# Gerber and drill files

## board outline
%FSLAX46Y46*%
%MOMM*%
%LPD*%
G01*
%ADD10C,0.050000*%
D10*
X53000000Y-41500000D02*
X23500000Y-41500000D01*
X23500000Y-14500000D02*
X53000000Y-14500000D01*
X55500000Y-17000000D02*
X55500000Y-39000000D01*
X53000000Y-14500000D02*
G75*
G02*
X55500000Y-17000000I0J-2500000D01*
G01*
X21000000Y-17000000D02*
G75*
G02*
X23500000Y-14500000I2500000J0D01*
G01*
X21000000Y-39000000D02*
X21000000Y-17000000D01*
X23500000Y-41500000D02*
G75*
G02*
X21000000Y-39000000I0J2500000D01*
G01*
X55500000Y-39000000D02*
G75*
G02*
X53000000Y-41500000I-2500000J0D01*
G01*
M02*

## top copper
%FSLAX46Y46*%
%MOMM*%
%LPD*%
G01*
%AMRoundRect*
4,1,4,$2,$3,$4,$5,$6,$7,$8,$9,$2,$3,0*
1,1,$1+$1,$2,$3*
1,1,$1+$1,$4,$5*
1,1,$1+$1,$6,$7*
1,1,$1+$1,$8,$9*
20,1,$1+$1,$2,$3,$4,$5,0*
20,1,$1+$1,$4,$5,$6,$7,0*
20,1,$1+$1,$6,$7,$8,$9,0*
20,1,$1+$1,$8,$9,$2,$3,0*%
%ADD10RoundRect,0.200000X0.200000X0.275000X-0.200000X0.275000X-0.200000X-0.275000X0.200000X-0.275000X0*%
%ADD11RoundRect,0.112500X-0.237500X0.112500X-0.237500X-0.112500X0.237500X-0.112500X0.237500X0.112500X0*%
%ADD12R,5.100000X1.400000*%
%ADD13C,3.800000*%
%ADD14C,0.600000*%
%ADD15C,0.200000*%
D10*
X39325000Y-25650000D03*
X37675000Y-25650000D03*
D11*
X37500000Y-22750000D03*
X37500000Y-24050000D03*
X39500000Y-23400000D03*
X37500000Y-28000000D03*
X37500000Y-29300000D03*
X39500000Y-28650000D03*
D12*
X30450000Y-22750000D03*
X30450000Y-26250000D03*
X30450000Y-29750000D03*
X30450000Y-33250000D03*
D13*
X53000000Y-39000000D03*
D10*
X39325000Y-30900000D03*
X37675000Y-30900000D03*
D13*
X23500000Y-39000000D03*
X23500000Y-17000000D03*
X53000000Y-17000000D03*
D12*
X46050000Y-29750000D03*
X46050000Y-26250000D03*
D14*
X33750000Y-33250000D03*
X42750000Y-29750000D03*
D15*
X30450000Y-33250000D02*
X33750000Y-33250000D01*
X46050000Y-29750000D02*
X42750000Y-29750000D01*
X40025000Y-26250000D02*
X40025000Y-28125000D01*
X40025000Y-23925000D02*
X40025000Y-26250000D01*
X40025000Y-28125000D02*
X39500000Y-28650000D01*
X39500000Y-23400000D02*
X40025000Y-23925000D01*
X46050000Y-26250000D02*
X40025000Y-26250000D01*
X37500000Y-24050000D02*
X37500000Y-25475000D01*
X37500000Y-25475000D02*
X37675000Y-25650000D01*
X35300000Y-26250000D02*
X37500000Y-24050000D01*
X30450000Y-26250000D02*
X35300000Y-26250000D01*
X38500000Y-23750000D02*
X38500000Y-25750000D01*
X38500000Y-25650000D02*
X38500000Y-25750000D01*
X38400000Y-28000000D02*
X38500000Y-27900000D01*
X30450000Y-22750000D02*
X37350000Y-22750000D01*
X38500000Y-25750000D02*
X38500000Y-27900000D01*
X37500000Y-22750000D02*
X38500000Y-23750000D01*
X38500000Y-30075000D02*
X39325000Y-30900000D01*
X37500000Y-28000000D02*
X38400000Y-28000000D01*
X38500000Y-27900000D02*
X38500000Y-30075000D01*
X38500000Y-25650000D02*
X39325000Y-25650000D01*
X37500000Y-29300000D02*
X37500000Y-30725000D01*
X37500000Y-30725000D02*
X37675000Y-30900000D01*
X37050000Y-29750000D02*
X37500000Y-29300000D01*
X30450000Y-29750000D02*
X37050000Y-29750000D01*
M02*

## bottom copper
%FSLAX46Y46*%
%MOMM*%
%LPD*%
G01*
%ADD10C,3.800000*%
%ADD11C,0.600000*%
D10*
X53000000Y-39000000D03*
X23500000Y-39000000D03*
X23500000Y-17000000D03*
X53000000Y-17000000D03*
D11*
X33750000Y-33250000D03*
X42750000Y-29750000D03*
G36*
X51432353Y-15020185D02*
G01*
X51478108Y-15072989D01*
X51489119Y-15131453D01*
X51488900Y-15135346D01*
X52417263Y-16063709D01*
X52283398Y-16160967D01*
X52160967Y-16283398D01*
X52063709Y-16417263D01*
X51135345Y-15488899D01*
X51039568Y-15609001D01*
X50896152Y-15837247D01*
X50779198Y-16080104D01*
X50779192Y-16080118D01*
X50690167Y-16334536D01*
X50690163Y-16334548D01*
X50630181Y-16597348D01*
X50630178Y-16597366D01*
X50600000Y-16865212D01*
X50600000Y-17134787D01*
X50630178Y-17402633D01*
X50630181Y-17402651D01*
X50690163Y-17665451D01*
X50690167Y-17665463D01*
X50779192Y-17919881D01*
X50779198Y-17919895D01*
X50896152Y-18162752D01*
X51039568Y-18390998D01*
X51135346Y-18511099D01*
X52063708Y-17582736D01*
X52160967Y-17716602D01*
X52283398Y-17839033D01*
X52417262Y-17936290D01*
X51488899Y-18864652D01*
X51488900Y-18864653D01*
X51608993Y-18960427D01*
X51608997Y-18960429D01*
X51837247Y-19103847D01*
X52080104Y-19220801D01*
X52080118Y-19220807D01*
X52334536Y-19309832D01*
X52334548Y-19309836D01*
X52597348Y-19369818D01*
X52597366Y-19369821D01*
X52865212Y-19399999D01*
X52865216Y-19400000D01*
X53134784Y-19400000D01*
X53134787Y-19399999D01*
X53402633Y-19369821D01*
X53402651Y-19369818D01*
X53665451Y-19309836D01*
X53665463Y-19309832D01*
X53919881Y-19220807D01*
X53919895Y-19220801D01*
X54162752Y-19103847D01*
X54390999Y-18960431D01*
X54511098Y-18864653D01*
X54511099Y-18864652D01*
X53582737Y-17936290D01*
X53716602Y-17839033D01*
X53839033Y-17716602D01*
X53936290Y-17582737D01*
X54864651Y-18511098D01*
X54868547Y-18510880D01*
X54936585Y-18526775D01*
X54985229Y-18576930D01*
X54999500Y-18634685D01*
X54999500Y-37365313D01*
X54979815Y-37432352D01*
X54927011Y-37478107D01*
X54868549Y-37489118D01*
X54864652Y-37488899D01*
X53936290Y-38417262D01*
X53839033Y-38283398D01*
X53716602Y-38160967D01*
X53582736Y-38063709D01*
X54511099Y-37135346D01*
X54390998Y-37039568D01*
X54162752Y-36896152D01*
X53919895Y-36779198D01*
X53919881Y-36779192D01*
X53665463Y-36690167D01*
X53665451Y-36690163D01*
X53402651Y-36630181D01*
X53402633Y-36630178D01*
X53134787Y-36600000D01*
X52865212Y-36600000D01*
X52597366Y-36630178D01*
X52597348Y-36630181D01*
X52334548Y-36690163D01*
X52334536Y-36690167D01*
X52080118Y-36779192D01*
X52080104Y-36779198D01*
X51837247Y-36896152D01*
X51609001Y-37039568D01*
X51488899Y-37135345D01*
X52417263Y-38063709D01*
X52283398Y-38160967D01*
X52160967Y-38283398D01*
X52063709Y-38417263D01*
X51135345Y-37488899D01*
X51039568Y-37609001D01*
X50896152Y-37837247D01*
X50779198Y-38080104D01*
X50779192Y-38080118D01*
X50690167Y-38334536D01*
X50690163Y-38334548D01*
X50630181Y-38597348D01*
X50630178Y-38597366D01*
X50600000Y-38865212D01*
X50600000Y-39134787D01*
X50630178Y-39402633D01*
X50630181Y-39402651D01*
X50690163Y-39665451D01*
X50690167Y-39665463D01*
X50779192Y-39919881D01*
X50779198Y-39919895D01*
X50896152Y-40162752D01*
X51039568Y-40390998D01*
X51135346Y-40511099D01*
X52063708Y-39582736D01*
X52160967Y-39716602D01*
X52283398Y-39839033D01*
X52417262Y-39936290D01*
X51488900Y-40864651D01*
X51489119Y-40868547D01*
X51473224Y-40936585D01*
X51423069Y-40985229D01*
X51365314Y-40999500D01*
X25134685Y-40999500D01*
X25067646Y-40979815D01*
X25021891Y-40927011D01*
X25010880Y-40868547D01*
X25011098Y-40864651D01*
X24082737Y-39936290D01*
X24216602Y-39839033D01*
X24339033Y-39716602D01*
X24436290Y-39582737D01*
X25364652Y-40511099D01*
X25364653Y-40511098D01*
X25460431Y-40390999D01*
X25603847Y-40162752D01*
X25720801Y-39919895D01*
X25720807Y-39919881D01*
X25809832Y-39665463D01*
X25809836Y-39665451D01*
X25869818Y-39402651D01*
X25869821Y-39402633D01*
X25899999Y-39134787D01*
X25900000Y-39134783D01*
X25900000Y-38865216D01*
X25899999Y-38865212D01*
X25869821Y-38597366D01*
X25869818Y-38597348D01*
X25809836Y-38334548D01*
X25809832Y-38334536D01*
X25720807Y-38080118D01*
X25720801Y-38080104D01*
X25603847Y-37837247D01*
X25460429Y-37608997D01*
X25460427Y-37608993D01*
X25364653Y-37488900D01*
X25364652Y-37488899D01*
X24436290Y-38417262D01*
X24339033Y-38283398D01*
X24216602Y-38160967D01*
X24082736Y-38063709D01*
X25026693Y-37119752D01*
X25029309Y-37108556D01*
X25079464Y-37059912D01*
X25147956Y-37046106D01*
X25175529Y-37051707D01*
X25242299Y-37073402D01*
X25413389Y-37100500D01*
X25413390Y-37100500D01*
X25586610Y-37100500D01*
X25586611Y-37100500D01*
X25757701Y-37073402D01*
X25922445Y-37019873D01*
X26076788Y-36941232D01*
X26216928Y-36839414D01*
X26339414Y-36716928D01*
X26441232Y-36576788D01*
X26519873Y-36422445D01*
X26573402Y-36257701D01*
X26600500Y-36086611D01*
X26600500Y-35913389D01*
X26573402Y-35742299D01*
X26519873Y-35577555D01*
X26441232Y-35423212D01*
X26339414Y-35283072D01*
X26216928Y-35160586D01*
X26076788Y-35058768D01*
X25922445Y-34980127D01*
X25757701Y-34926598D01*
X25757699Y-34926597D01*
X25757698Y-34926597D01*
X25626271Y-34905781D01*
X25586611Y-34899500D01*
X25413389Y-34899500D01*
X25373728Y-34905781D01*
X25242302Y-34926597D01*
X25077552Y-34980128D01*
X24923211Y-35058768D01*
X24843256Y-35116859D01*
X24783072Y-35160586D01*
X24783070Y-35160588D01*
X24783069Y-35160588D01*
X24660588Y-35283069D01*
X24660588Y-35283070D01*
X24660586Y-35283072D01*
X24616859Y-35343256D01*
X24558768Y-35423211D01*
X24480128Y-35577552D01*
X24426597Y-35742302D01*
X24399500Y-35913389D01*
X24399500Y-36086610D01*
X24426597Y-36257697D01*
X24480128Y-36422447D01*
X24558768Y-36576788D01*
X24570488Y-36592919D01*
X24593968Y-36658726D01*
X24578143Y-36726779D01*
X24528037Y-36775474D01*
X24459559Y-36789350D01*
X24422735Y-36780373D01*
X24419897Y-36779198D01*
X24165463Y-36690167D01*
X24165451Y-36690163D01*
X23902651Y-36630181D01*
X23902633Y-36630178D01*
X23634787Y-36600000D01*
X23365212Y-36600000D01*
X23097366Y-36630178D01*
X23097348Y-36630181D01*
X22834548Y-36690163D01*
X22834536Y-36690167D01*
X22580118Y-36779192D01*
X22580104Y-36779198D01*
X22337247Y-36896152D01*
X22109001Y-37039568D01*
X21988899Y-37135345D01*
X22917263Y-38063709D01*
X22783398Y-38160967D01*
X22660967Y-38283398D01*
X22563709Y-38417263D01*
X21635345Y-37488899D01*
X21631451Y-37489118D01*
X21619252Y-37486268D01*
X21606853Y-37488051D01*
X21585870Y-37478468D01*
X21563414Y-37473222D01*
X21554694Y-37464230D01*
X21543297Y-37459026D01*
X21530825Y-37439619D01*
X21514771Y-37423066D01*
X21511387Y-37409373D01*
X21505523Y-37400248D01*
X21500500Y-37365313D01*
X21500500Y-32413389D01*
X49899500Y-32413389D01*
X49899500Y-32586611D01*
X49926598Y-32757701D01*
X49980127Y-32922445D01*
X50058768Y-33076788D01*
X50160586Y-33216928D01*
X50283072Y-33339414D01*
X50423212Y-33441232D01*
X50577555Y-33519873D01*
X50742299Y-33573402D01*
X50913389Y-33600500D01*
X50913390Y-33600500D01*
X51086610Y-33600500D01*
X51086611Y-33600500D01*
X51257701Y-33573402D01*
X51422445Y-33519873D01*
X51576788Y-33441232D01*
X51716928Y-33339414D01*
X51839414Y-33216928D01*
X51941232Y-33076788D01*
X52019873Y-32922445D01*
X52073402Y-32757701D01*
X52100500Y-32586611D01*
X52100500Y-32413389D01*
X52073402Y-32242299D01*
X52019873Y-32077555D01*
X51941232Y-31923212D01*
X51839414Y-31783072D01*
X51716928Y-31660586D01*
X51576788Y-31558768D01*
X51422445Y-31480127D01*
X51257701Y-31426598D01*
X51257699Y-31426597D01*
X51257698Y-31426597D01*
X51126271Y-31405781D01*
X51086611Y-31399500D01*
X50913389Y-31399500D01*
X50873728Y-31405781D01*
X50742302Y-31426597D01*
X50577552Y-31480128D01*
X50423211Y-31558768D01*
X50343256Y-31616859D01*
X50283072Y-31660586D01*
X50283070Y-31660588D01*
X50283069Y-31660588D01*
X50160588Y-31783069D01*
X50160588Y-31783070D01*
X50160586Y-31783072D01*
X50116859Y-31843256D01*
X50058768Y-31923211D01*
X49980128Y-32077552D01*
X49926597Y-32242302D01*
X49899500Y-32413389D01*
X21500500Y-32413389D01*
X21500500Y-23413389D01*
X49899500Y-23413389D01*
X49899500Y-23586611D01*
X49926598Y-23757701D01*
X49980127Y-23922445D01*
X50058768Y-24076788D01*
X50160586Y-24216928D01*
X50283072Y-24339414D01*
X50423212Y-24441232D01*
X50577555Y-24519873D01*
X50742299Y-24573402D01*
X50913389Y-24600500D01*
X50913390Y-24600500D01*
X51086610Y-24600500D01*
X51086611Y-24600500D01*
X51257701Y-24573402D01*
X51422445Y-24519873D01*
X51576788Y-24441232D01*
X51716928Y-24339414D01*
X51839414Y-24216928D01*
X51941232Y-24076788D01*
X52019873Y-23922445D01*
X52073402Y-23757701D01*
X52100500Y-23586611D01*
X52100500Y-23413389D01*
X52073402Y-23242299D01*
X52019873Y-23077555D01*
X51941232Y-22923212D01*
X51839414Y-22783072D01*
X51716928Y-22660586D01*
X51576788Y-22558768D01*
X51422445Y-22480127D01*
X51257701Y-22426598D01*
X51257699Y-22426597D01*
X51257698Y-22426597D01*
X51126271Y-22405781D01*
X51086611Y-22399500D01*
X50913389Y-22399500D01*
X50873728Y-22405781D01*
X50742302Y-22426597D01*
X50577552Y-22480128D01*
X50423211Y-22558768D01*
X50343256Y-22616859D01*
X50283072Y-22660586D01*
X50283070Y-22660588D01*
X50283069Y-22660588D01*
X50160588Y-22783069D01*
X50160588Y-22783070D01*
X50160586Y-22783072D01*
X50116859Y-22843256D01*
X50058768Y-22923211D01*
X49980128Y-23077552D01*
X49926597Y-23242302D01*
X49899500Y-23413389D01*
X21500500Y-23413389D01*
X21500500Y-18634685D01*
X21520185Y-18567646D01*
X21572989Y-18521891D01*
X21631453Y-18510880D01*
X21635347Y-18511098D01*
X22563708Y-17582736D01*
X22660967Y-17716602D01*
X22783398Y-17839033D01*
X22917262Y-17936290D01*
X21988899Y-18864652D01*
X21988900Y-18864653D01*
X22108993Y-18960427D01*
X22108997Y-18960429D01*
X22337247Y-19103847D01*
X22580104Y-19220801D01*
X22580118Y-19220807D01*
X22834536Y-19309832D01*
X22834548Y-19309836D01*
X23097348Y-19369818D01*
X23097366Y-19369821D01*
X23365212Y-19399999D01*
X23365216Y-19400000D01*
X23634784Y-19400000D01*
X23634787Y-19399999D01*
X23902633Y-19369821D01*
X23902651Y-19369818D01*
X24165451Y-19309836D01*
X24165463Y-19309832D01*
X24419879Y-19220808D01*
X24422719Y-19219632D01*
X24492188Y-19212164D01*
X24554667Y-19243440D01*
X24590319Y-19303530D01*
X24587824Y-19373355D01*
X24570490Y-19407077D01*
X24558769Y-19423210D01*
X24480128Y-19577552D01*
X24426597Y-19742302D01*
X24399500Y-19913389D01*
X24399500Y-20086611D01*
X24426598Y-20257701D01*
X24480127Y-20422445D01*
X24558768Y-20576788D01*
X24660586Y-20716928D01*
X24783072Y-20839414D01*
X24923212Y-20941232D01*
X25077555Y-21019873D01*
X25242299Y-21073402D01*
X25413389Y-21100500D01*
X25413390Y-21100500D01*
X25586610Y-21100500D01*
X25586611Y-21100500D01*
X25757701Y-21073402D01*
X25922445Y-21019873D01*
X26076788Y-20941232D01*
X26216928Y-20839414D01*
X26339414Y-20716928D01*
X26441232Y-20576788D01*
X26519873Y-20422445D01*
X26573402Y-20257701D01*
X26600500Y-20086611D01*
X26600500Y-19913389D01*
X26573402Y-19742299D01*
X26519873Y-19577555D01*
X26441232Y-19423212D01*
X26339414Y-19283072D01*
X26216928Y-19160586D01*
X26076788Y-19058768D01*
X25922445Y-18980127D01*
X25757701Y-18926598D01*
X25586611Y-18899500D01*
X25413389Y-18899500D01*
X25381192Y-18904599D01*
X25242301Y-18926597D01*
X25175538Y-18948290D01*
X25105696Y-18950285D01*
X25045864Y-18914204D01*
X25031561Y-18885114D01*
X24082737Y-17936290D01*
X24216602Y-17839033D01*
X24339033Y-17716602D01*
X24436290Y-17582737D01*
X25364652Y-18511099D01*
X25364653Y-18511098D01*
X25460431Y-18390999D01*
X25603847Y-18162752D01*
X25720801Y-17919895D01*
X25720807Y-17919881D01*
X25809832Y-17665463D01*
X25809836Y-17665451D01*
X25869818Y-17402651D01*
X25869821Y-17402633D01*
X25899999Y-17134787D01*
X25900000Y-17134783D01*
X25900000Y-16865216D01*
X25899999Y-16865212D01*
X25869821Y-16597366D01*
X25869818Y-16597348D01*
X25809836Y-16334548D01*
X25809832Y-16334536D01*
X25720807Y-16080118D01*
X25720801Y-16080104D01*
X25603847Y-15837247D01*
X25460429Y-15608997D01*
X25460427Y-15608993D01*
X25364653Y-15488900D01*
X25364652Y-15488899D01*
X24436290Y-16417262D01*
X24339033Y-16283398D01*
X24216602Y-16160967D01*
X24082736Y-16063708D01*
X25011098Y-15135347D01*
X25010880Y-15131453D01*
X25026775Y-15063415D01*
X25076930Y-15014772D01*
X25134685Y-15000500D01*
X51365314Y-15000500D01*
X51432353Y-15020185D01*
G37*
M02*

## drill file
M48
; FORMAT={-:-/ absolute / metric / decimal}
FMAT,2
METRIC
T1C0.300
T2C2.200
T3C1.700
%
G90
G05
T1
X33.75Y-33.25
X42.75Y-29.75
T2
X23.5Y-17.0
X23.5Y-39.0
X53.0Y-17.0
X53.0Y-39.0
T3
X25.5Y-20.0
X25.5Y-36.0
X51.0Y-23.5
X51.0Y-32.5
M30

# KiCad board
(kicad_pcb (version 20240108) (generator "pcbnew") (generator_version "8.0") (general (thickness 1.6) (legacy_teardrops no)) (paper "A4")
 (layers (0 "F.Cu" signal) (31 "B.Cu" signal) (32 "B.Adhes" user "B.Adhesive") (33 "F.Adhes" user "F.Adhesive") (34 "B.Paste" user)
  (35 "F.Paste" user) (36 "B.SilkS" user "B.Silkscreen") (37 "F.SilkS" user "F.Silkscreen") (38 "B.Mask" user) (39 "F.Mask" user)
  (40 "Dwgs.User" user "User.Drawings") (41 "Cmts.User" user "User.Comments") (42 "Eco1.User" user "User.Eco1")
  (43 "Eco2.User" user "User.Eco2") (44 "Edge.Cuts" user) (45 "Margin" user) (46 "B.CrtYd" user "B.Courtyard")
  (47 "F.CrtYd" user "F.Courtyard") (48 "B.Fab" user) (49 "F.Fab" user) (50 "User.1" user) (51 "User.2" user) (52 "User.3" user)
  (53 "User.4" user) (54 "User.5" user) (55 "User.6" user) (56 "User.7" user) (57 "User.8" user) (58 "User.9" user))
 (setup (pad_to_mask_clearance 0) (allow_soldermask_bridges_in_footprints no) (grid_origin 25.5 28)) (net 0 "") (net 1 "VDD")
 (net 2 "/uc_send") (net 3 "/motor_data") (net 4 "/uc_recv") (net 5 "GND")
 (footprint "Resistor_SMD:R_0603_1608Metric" (layer "F.Cu") (at 38.5 25.65 180)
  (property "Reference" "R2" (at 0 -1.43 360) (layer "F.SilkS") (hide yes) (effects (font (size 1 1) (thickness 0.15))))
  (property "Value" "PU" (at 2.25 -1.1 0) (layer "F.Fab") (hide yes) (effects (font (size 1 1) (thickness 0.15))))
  (pad "1" smd roundrect (at -0.825 0 180) (size 0.8 0.95) (layers "F.Cu" "F.Paste" "F.Mask") (roundrect_rratio 0.25) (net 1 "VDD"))
  (pad "2" smd roundrect (at 0.825 0 180) (size 0.8 0.95) (layers "F.Cu" "F.Paste" "F.Mask") (roundrect_rratio 0.25) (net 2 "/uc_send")))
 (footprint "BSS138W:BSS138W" (layer "F.Cu") (at 38.5 23.4)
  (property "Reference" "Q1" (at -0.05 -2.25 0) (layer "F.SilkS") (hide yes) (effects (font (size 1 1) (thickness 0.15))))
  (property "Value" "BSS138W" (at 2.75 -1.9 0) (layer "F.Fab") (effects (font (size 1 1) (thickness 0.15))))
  (pad "1" smd roundrect (at -1 -0.65 270) (size 0.45 0.7) (layers "F.Cu" "F.Paste" "F.Mask") (roundrect_rratio 0.25) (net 1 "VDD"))
  (pad "2" smd roundrect (at -1 0.65 270) (size 0.45 0.7) (layers "F.Cu" "F.Paste" "F.Mask") (roundrect_rratio 0.25) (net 2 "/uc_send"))
  (pad "3" smd roundrect (at 1 0 270) (size 0.45 0.7) (layers "F.Cu" "F.Paste" "F.Mask") (roundrect_rratio 0.25) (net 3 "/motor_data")))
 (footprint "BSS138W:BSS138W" (layer "F.Cu") (at 38.5 28.65)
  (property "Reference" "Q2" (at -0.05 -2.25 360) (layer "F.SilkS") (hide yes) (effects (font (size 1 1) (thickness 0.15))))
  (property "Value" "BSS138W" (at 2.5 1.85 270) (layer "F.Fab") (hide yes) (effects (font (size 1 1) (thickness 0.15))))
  (pad "1" smd roundrect (at -1 -0.65 270) (size 0.45 0.7) (layers "F.Cu" "F.Paste" "F.Mask") (roundrect_rratio 0.25) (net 1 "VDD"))
  (pad "2" smd roundrect (at -1 0.65 270) (size 0.45 0.7) (layers "F.Cu" "F.Paste" "F.Mask") (roundrect_rratio 0.25) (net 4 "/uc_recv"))
  (pad "3" smd roundrect (at 1 0 270) (size 0.45 0.7) (layers "F.Cu" "F.Paste" "F.Mask") (roundrect_rratio 0.25) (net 3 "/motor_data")))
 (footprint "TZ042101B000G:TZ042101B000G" (layer "F.Cu") (at 25.5 28 -90)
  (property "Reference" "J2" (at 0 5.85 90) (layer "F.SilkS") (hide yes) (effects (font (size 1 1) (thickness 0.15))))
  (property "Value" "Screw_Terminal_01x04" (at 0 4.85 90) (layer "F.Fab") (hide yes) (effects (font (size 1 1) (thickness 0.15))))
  (pad "" np_thru_hole circle (at -8 0 270) (size 1.7 1.7) (drill 1.7) (layers "*.Cu" "*.Mask"))
  (pad "" np_thru_hole circle (at 8 0 270) (size 1.7 1.7) (drill 1.7) (layers "*.Cu" "*.Mask"))
  (pad "1" smd rect (at -5.25 -4.95 270) (size 1.4 5.1) (layers "F.Cu" "F.Paste" "F.Mask") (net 1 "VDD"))
  (pad "2" smd rect (at -1.75 -4.95 270) (size 1.4 5.1) (layers "F.Cu" "F.Paste" "F.Mask") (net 2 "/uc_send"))
  (pad "3" smd rect (at 1.75 -4.95 270) (size 1.4 5.1) (layers "F.Cu" "F.Paste" "F.Mask") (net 4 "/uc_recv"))
  (pad "4" smd rect (at 5.25 -4.95 270) (size 1.4 5.1) (layers "F.Cu" "F.Paste" "F.Mask") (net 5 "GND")))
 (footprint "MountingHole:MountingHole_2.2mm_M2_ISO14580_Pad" (layer "F.Cu") (at 53 39)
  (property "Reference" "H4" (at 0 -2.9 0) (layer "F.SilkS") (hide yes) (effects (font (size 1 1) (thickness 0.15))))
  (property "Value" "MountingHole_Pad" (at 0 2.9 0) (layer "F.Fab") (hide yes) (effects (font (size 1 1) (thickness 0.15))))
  (pad "1" thru_hole circle (at 0 0) (size 3.8 3.8) (drill 2.2) (layers "*.Cu" "*.Mask") (remove_unused_layers no) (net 5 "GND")))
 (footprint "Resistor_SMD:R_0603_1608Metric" (layer "F.Cu") (at 38.5 30.9 180)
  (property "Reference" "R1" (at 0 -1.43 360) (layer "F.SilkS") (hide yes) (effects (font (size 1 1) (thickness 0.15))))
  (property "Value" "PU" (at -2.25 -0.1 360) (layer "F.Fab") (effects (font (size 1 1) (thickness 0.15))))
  (pad "1" smd roundrect (at -0.825 0 180) (size 0.8 0.95) (layers "F.Cu" "F.Paste" "F.Mask") (roundrect_rratio 0.25) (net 1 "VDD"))
  (pad "2" smd roundrect (at 0.825 0 180) (size 0.8 0.95) (layers "F.Cu" "F.Paste" "F.Mask") (roundrect_rratio 0.25) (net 4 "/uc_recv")))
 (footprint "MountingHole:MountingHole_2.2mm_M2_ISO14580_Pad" (layer "F.Cu") (at 23.5 39)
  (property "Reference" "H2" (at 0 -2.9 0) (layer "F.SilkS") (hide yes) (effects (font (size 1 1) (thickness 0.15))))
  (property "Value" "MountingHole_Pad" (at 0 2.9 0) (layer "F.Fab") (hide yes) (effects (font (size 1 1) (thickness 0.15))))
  (pad "1" thru_hole circle (at 0 0) (size 3.8 3.8) (drill 2.2) (layers "*.Cu" "*.Mask") (remove_unused_layers no) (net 5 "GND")))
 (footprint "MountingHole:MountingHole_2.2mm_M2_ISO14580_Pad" (layer "F.Cu") (at 23.5 17)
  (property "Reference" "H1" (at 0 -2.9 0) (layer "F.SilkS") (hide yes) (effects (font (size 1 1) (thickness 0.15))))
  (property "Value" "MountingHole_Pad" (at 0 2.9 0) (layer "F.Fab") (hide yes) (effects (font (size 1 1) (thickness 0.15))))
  (pad "1" thru_hole circle (at 0 0) (size 3.8 3.8) (drill 2.2) (layers "*.Cu" "*.Mask") (remove_unused_layers no) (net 5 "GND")))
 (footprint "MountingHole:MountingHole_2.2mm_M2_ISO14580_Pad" (layer "F.Cu") (at 53 17)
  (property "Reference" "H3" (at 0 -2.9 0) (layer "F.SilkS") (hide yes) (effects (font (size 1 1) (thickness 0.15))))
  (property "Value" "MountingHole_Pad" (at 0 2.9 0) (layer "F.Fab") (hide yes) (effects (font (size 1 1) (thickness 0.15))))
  (pad "1" thru_hole circle (at 0 0) (size 3.8 3.8) (drill 2.2) (layers "*.Cu" "*.Mask") (remove_unused_layers no) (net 5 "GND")))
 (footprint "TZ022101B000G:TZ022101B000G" (layer "F.Cu") (at 51 28 90)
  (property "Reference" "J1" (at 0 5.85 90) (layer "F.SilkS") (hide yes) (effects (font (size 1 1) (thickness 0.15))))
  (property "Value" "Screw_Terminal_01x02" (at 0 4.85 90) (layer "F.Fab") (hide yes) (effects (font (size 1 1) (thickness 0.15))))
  (pad "" np_thru_hole circle (at -4.5 0 90) (size 1.7 1.7) (drill 1.7) (layers "*.Cu" "*.Mask"))
  (pad "" np_thru_hole circle (at 4.5 0 90) (size 1.7 1.7) (drill 1.7) (layers "*.Cu" "*.Mask"))
  (pad "1" smd rect (at -1.75 -4.95 90) (size 1.4 5.1) (layers "F.Cu" "F.Paste" "F.Mask") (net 5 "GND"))
  (pad "2" smd rect (at 1.75 -4.95 90) (size 1.4 5.1) (layers "F.Cu" "F.Paste" "F.Mask") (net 3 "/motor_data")))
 (gr_line (start 53 41.5) (end 23.5 41.5) (stroke (width 0.05) (type default)) (layer "Edge.Cuts"))
 (gr_line (start 23.5 14.5) (end 53 14.5) (stroke (width 0.05) (type default)) (layer "Edge.Cuts"))
 (gr_line (start 55.5 17) (end 55.5 39) (stroke (width 0.05) (type default)) (layer "Edge.Cuts"))
 (gr_arc (start 53 14.5) (mid 54.767767 15.232233) (end 55.5 17) (stroke (width 0.05) (type default)) (layer "Edge.Cuts"))
 (gr_arc (start 21 17) (mid 21.732233 15.232233) (end 23.5 14.5) (stroke (width 0.05) (type default)) (layer "Edge.Cuts"))
 (gr_line (start 21 39) (end 21 17) (stroke (width 0.05) (type default)) (layer "Edge.Cuts"))
 (gr_arc (start 23.5 41.5) (mid 21.732233 40.767767) (end 21 39) (stroke (width 0.05) (type default)) (layer "Edge.Cuts"))
 (gr_arc (start 55.5 39) (mid 54.767767 40.767767) (end 53 41.5) (stroke (width 0.05) (type default)) (layer "Edge.Cuts"))
 (segment (start 30.45 33.25) (end 33.75 33.25) (width 0.2) (layer "F.Cu") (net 5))
 (segment (start 46.05 29.75) (end 42.75 29.75) (width 0.2) (layer "F.Cu") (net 5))
 (via (at 33.75 33.25) (size 0.6) (drill 0.3) (layers "F.Cu" "B.Cu") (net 5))
 (via (at 42.75 29.75) (size 0.6) (drill 0.3) (layers "F.Cu" "B.Cu") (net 5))
 (segment (start 40.025 26.25) (end 40.025 28.125) (width 0.2) (layer "F.Cu") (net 3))
 (segment (start 40.025 23.925) (end 40.025 26.25) (width 0.2) (layer "F.Cu") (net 3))
 (segment (start 40.025 28.125) (end 39.5 28.65) (width 0.2) (layer "F.Cu") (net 3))
 (segment (start 39.5 23.4) (end 40.025 23.925) (width 0.2) (layer "F.Cu") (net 3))
 (segment (start 46.05 26.25) (end 40.025 26.25) (width 0.2) (layer "F.Cu") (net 3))
 (segment (start 37.5 24.05) (end 37.5 25.475) (width 0.2) (layer "F.Cu") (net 2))
 (segment (start 37.5 25.475) (end 37.675 25.65) (width 0.2) (layer "F.Cu") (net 2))
 (segment (start 35.3 26.25) (end 37.5 24.05) (width 0.2) (layer "F.Cu") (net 2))
 (segment (start 30.45 26.25) (end 35.3 26.25) (width 0.2) (layer "F.Cu") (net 2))
 (segment (start 38.5 23.75) (end 38.5 25.75) (width 0.2) (layer "F.Cu") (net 1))
 (segment (start 38.5 25.65) (end 38.5 25.75) (width 0.2) (layer "F.Cu") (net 1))
 (segment (start 38.4 28) (end 38.5 27.9) (width 0.2) (layer "F.Cu") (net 1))
 (segment (start 30.45 22.75) (end 37.35 22.75) (width 0.2) (layer "F.Cu") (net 1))
 (segment (start 38.5 25.75) (end 38.5 27.9) (width 0.2) (layer "F.Cu") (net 1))
 (segment (start 37.5 22.75) (end 38.5 23.75) (width 0.2) (layer "F.Cu") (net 1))
 (segment (start 38.5 30.075) (end 39.325 30.9) (width 0.2) (layer "F.Cu") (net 1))
 (segment (start 37.5 28) (end 38.4 28) (width 0.2) (layer "F.Cu") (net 1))
 (segment (start 38.5 27.9) (end 38.5 30.075) (width 0.2) (layer "F.Cu") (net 1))
 (segment (start 38.5 25.65) (end 39.325 25.65) (width 0.2) (layer "F.Cu") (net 1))
 (segment (start 37.5 29.3) (end 37.5 30.725) (width 0.2) (layer "F.Cu") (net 4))
 (segment (start 37.5 30.725) (end 37.675 30.9) (width 0.2) (layer "F.Cu") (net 4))
 (segment (start 37.05 29.75) (end 37.5 29.3) (width 0.2) (layer "F.Cu") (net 4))
 (segment (start 30.45 29.75) (end 37.05 29.75) (width 0.2) (layer "F.Cu") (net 4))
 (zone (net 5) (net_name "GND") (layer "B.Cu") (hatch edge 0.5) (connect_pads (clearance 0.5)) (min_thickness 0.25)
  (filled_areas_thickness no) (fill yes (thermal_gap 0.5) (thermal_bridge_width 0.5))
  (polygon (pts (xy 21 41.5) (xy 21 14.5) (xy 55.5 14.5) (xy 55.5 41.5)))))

